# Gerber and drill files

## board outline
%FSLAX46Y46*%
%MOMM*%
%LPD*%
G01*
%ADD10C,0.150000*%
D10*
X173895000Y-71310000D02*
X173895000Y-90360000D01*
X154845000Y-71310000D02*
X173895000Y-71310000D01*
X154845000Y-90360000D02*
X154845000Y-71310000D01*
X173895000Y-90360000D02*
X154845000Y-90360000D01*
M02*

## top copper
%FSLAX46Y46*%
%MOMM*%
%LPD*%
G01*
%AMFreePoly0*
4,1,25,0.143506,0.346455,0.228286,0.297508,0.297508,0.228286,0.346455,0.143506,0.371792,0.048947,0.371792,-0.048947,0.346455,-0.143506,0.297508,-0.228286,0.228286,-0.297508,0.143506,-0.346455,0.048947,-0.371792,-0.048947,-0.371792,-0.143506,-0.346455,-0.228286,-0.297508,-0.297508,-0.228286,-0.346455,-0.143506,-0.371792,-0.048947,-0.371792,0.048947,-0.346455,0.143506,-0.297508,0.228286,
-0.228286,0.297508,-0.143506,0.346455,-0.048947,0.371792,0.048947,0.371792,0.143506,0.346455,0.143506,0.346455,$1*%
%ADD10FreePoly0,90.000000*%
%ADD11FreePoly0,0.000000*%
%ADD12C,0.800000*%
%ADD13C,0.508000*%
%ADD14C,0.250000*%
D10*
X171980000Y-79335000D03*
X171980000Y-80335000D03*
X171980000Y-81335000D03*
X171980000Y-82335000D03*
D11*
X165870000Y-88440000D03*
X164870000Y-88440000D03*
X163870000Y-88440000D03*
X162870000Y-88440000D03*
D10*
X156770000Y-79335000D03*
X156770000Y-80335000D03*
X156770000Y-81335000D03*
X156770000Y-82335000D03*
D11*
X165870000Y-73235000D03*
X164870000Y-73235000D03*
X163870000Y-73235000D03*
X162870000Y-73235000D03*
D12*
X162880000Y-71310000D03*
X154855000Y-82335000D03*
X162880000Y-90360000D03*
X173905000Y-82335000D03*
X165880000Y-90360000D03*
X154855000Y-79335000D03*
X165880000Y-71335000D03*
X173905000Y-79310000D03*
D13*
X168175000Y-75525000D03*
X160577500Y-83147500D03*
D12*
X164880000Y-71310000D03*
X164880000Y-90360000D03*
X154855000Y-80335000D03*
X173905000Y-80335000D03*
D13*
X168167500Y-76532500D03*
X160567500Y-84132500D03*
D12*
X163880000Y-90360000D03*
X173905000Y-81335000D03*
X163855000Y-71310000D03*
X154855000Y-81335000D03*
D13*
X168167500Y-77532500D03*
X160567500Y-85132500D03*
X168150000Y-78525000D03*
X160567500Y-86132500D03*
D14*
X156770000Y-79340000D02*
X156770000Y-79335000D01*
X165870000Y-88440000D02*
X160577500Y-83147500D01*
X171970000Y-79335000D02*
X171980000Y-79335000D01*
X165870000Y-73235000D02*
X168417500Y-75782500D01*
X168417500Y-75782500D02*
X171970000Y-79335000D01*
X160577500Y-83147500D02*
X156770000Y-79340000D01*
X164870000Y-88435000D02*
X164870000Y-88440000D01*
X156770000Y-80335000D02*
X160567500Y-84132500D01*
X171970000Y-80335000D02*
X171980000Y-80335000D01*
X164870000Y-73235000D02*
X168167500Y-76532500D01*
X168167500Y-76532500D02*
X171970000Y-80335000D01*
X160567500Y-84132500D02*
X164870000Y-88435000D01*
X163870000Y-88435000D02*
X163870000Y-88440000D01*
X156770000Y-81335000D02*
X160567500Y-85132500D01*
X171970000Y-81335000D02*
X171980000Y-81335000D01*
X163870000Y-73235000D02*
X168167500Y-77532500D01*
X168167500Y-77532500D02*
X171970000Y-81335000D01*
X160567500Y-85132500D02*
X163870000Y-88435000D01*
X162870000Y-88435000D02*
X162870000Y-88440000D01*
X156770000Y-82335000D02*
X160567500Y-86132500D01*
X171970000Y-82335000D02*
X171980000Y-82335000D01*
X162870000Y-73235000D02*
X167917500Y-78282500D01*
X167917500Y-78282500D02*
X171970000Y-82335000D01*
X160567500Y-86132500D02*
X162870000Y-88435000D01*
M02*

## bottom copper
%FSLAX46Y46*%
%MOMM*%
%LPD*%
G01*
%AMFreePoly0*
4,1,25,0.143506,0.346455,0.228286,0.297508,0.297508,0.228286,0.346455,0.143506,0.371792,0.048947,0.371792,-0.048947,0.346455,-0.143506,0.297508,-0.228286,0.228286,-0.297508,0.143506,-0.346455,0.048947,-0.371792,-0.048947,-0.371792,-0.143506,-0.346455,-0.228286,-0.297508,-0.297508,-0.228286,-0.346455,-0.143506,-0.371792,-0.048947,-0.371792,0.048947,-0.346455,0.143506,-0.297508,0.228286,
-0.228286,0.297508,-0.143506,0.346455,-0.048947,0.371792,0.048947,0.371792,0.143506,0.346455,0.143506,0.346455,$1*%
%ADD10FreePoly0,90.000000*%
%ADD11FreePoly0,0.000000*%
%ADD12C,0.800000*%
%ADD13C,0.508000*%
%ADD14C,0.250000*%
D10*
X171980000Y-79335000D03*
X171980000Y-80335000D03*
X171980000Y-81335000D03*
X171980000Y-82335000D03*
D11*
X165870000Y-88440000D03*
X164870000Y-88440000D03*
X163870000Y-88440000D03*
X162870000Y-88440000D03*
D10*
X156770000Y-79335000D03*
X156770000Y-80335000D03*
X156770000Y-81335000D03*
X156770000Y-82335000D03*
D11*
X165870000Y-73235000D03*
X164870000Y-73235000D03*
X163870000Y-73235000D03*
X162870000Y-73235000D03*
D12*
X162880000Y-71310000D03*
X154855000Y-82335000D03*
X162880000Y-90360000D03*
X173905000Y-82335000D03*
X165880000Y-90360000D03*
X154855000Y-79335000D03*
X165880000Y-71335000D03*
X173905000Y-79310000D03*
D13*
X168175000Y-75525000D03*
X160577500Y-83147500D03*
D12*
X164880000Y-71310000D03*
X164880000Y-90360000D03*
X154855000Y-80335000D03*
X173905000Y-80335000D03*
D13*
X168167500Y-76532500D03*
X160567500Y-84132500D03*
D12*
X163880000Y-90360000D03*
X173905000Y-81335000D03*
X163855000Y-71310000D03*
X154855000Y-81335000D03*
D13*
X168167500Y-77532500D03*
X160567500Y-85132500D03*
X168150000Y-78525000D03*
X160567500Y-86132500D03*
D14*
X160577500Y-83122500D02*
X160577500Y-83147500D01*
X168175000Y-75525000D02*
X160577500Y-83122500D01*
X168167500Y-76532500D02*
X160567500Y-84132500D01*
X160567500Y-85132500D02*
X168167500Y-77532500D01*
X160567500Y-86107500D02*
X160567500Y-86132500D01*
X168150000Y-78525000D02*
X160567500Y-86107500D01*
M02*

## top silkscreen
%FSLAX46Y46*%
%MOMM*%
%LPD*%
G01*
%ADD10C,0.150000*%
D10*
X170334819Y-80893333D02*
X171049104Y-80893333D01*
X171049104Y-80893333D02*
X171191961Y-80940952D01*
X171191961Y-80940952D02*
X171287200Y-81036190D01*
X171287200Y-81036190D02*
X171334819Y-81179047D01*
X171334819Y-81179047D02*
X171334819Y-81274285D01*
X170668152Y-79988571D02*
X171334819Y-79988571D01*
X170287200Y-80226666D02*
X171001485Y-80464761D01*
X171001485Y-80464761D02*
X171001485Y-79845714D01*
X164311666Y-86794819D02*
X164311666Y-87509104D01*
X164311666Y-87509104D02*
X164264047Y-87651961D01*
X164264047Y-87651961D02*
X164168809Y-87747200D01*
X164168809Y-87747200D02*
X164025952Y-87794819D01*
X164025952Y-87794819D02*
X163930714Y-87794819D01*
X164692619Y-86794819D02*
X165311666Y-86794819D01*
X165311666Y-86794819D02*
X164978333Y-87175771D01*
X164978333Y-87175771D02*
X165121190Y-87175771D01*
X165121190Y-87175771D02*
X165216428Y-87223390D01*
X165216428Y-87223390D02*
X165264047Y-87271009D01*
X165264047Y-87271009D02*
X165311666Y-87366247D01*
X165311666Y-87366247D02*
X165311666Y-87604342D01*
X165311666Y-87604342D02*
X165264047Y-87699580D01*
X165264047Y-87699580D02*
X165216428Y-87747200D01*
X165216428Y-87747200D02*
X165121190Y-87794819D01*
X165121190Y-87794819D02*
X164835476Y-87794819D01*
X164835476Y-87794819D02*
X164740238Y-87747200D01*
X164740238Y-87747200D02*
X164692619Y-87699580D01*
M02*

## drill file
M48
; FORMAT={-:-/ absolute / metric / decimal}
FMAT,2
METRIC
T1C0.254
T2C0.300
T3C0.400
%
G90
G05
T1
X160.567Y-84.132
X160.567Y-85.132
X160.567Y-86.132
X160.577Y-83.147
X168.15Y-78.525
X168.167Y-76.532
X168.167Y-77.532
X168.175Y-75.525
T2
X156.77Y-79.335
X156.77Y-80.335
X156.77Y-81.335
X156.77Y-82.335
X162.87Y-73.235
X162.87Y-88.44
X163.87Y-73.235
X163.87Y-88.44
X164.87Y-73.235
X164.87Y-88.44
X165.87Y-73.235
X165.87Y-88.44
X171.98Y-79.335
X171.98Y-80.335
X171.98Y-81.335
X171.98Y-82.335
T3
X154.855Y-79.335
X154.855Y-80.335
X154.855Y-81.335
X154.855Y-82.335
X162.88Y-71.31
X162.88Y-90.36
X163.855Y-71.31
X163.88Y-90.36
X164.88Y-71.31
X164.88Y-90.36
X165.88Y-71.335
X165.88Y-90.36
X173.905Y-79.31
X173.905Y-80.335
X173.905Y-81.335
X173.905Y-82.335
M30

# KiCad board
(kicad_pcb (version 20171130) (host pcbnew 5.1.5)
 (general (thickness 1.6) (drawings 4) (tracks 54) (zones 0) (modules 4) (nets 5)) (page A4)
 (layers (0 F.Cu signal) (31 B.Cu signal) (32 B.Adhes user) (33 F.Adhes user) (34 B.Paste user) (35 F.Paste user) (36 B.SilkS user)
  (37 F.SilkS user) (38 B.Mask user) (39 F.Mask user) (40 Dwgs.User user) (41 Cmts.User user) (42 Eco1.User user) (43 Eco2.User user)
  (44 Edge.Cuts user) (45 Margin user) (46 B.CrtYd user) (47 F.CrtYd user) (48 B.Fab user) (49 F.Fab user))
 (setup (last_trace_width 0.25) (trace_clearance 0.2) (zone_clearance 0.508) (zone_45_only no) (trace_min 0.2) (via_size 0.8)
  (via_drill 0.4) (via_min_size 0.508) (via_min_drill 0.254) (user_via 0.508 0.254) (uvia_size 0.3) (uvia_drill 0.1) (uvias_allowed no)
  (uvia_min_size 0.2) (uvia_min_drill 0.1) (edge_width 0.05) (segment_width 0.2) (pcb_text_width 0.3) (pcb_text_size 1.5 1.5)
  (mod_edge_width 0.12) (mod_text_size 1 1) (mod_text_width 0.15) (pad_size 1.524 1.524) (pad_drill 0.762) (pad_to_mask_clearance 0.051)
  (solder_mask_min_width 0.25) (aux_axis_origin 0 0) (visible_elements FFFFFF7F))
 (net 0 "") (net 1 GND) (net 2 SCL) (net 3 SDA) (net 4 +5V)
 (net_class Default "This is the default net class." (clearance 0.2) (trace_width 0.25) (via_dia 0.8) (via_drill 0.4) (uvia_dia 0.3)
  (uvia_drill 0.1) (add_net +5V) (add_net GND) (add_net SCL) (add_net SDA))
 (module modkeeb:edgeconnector (layer F.Cu) (at 173.98 80.835 90)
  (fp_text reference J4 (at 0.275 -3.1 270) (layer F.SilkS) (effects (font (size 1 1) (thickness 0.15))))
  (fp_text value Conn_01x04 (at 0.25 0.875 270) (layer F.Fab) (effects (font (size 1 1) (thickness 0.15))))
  (pad 4 thru_hole custom (at 1.5 -2 90) (size 0.75 0.75) (drill 0.3) (layers *.Cu *.Mask) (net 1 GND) (zone_connect 0)
   (options (clearance outline) (anchor circle)) (primitives))
  (pad 3 thru_hole custom (at 0.5 -2 90) (size 0.75 0.75) (drill 0.3) (layers *.Cu *.Mask) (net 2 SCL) (zone_connect 0)
   (options (clearance outline) (anchor circle)) (primitives))
  (pad 2 thru_hole custom (at -0.5 -2 90) (size 0.75 0.75) (drill 0.3) (layers *.Cu *.Mask) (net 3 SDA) (zone_connect 0)
   (options (clearance outline) (anchor circle)) (primitives))
  (pad 1 thru_hole custom (at -1.5 -2 90) (size 0.75 0.75) (drill 0.3) (layers *.Cu *.Mask) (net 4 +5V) (zone_connect 0)
   (options (clearance outline) (anchor circle)) (primitives)))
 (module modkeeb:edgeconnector (layer F.Cu) (at 164.37 90.44)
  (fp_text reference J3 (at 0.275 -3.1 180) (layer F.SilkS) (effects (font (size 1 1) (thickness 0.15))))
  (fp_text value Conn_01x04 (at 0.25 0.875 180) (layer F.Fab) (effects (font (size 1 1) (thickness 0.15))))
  (pad 4 thru_hole custom (at 1.5 -2) (size 0.75 0.75) (drill 0.3) (layers *.Cu *.Mask) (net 1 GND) (zone_connect 0)
   (options (clearance outline) (anchor circle)) (primitives))
  (pad 3 thru_hole custom (at 0.5 -2) (size 0.75 0.75) (drill 0.3) (layers *.Cu *.Mask) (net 2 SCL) (zone_connect 0)
   (options (clearance outline) (anchor circle)) (primitives))
  (pad 2 thru_hole custom (at -0.5 -2) (size 0.75 0.75) (drill 0.3) (layers *.Cu *.Mask) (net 3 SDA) (zone_connect 0)
   (options (clearance outline) (anchor circle)) (primitives))
  (pad 1 thru_hole custom (at -1.5 -2) (size 0.75 0.75) (drill 0.3) (layers *.Cu *.Mask) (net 4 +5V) (zone_connect 0)
   (options (clearance outline) (anchor circle)) (primitives)))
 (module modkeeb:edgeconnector (layer B.Cu) (at 154.77 80.835 90)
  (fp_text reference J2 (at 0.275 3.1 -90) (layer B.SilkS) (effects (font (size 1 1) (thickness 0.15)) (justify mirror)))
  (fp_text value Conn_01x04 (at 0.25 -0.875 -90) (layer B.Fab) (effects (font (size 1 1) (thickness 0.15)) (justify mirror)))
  (pad 4 thru_hole custom (at 1.5 2 90) (size 0.75 0.75) (drill 0.3) (layers *.Cu *.Mask) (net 1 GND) (zone_connect 0)
   (options (clearance outline) (anchor circle)) (primitives))
  (pad 3 thru_hole custom (at 0.5 2 90) (size 0.75 0.75) (drill 0.3) (layers *.Cu *.Mask) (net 2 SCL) (zone_connect 0)
   (options (clearance outline) (anchor circle)) (primitives))
  (pad 2 thru_hole custom (at -0.5 2 90) (size 0.75 0.75) (drill 0.3) (layers *.Cu *.Mask) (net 3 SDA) (zone_connect 0)
   (options (clearance outline) (anchor circle)) (primitives))
  (pad 1 thru_hole custom (at -1.5 2 90) (size 0.75 0.75) (drill 0.3) (layers *.Cu *.Mask) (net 4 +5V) (zone_connect 0)
   (options (clearance outline) (anchor circle)) (primitives)))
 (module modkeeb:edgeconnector (layer B.Cu) (at 164.37 71.235)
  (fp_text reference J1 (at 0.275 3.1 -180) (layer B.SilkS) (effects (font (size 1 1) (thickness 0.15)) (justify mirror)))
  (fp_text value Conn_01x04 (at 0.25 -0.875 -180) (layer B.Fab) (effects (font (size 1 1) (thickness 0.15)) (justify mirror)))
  (pad 4 thru_hole custom (at 1.5 2) (size 0.75 0.75) (drill 0.3) (layers *.Cu *.Mask) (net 1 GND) (zone_connect 0)
   (options (clearance outline) (anchor circle)) (primitives))
  (pad 3 thru_hole custom (at 0.5 2) (size 0.75 0.75) (drill 0.3) (layers *.Cu *.Mask) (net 2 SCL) (zone_connect 0)
   (options (clearance outline) (anchor circle)) (primitives))
  (pad 2 thru_hole custom (at -0.5 2) (size 0.75 0.75) (drill 0.3) (layers *.Cu *.Mask) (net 3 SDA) (zone_connect 0)
   (options (clearance outline) (anchor circle)) (primitives))
  (pad 1 thru_hole custom (at -1.5 2) (size 0.75 0.75) (drill 0.3) (layers *.Cu *.Mask) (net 4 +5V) (zone_connect 0)
   (options (clearance outline) (anchor circle)) (primitives)))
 (gr_line (start 173.895 71.31) (end 173.895 90.36) (layer Edge.Cuts) (width 0.15))
 (gr_line (start 154.845 71.31) (end 173.895 71.31) (layer Edge.Cuts) (width 0.15))
 (gr_line (start 154.845 90.36) (end 154.845 71.31) (layer Edge.Cuts) (width 0.15))
 (gr_line (start 173.895 90.36) (end 154.845 90.36) (layer Edge.Cuts) (width 0.15))
 (via (at 162.88 71.31) (size 0.8) (drill 0.4) (layers F.Cu B.Cu) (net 4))
 (via (at 154.855 82.335) (size 0.8) (drill 0.4) (layers F.Cu B.Cu) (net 4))
 (via (at 162.88 90.36) (size 0.8) (drill 0.4) (layers F.Cu B.Cu) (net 4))
 (via (at 173.905 82.335) (size 0.8) (drill 0.4) (layers F.Cu B.Cu) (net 4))
 (via (at 165.88 90.36) (size 0.8) (drill 0.4) (layers F.Cu B.Cu) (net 1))
 (via (at 154.855 79.335) (size 0.8) (drill 0.4) (layers F.Cu B.Cu) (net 1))
 (via (at 165.88 71.335) (size 0.8) (drill 0.4) (layers F.Cu B.Cu) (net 1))
 (via (at 173.905 79.31) (size 0.8) (drill 0.4) (layers F.Cu B.Cu) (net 1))
 (segment (start 156.77 79.34) (end 156.77 79.335) (width 0.25) (layer F.Cu) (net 1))
 (segment (start 165.87 88.44) (end 160.5775 83.1475) (width 0.25) (layer F.Cu) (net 1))
 (segment (start 171.97 79.335) (end 171.98 79.335) (width 0.25) (layer F.Cu) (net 1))
 (segment (start 165.87 73.235) (end 168.4175 75.7825) (width 0.25) (layer F.Cu) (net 1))
 (segment (start 168.4175 75.7825) (end 171.97 79.335) (width 0.25) (layer F.Cu) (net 1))
 (via (at 168.175 75.525) (size 0.508) (drill 0.254) (layers F.Cu B.Cu) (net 1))
 (segment (start 160.5775 83.1475) (end 156.77 79.34) (width 0.25) (layer F.Cu) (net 1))
 (via (at 160.5775 83.1475) (size 0.508) (drill 0.254) (layers F.Cu B.Cu) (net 1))
 (segment (start 160.5775 83.1225) (end 160.5775 83.1475) (width 0.25) (layer B.Cu) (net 1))
 (segment (start 168.175 75.525) (end 160.5775 83.1225) (width 0.25) (layer B.Cu) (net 1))
 (via (at 164.88 71.31) (size 0.8) (drill 0.4) (layers F.Cu B.Cu) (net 2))
 (via (at 164.88 90.36) (size 0.8) (drill 0.4) (layers F.Cu B.Cu) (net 2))
 (via (at 154.855 80.335) (size 0.8) (drill 0.4) (layers F.Cu B.Cu) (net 2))
 (via (at 173.905 80.335) (size 0.8) (drill 0.4) (layers F.Cu B.Cu) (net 2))
 (segment (start 164.87 88.435) (end 164.87 88.44) (width 0.25) (layer F.Cu) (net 2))
 (segment (start 156.77 80.335) (end 160.5675 84.1325) (width 0.25) (layer F.Cu) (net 2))
 (segment (start 171.97 80.335) (end 171.98 80.335) (width 0.25) (layer F.Cu) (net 2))
 (segment (start 164.87 73.235) (end 168.1675 76.5325) (width 0.25) (layer F.Cu) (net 2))
 (segment (start 168.1675 76.5325) (end 171.97 80.335) (width 0.25) (layer F.Cu) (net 2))
 (via (at 168.1675 76.5325) (size 0.508) (drill 0.254) (layers F.Cu B.Cu) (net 2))
 (segment (start 160.5675 84.1325) (end 164.87 88.435) (width 0.25) (layer F.Cu) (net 2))
 (via (at 160.5675 84.1325) (size 0.508) (drill 0.254) (layers F.Cu B.Cu) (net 2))
 (segment (start 168.1675 76.5325) (end 160.5675 84.1325) (width 0.25) (layer B.Cu) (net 2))
 (via (at 163.88 90.36) (size 0.8) (drill 0.4) (layers F.Cu B.Cu) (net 3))
 (via (at 173.905 81.335) (size 0.8) (drill 0.4) (layers F.Cu B.Cu) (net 3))
 (via (at 163.855 71.31) (size 0.8) (drill 0.4) (layers F.Cu B.Cu) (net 3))
 (via (at 154.855 81.335) (size 0.8) (drill 0.4) (layers F.Cu B.Cu) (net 3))
 (segment (start 163.87 88.435) (end 163.87 88.44) (width 0.25) (layer F.Cu) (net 3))
 (segment (start 156.77 81.335) (end 160.5675 85.1325) (width 0.25) (layer F.Cu) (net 3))
 (segment (start 171.97 81.335) (end 171.98 81.335) (width 0.25) (layer F.Cu) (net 3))
 (segment (start 163.87 73.235) (end 168.1675 77.5325) (width 0.25) (layer F.Cu) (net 3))
 (segment (start 168.1675 77.5325) (end 171.97 81.335) (width 0.25) (layer F.Cu) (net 3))
 (via (at 168.1675 77.5325) (size 0.508) (drill 0.254) (layers F.Cu B.Cu) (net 3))
 (segment (start 160.5675 85.1325) (end 163.87 88.435) (width 0.25) (layer F.Cu) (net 3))
 (via (at 160.5675 85.1325) (size 0.508) (drill 0.254) (layers F.Cu B.Cu) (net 3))
 (segment (start 160.5675 85.1325) (end 168.1675 77.5325) (width 0.25) (layer B.Cu) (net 3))
 (segment (start 162.87 88.435) (end 162.87 88.44) (width 0.25) (layer F.Cu) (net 4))
 (segment (start 156.77 82.335) (end 160.5675 86.1325) (width 0.25) (layer F.Cu) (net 4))
 (segment (start 171.97 82.335) (end 171.98 82.335) (width 0.25) (layer F.Cu) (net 4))
 (segment (start 162.87 73.235) (end 167.9175 78.2825) (width 0.25) (layer F.Cu) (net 4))
 (segment (start 167.9175 78.2825) (end 171.97 82.335) (width 0.25) (layer F.Cu) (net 4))
 (via (at 168.15 78.525) (size 0.508) (drill 0.254) (layers F.Cu B.Cu) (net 4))
 (segment (start 160.5675 86.1325) (end 162.87 88.435) (width 0.25) (layer F.Cu) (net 4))
 (via (at 160.5675 86.1325) (size 0.508) (drill 0.254) (layers F.Cu B.Cu) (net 4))
 (segment (start 160.5675 86.1075) (end 160.5675 86.1325) (width 0.25) (layer B.Cu) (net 4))
 (segment (start 168.15 78.525) (end 160.5675 86.1075) (width 0.25) (layer B.Cu) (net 4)))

